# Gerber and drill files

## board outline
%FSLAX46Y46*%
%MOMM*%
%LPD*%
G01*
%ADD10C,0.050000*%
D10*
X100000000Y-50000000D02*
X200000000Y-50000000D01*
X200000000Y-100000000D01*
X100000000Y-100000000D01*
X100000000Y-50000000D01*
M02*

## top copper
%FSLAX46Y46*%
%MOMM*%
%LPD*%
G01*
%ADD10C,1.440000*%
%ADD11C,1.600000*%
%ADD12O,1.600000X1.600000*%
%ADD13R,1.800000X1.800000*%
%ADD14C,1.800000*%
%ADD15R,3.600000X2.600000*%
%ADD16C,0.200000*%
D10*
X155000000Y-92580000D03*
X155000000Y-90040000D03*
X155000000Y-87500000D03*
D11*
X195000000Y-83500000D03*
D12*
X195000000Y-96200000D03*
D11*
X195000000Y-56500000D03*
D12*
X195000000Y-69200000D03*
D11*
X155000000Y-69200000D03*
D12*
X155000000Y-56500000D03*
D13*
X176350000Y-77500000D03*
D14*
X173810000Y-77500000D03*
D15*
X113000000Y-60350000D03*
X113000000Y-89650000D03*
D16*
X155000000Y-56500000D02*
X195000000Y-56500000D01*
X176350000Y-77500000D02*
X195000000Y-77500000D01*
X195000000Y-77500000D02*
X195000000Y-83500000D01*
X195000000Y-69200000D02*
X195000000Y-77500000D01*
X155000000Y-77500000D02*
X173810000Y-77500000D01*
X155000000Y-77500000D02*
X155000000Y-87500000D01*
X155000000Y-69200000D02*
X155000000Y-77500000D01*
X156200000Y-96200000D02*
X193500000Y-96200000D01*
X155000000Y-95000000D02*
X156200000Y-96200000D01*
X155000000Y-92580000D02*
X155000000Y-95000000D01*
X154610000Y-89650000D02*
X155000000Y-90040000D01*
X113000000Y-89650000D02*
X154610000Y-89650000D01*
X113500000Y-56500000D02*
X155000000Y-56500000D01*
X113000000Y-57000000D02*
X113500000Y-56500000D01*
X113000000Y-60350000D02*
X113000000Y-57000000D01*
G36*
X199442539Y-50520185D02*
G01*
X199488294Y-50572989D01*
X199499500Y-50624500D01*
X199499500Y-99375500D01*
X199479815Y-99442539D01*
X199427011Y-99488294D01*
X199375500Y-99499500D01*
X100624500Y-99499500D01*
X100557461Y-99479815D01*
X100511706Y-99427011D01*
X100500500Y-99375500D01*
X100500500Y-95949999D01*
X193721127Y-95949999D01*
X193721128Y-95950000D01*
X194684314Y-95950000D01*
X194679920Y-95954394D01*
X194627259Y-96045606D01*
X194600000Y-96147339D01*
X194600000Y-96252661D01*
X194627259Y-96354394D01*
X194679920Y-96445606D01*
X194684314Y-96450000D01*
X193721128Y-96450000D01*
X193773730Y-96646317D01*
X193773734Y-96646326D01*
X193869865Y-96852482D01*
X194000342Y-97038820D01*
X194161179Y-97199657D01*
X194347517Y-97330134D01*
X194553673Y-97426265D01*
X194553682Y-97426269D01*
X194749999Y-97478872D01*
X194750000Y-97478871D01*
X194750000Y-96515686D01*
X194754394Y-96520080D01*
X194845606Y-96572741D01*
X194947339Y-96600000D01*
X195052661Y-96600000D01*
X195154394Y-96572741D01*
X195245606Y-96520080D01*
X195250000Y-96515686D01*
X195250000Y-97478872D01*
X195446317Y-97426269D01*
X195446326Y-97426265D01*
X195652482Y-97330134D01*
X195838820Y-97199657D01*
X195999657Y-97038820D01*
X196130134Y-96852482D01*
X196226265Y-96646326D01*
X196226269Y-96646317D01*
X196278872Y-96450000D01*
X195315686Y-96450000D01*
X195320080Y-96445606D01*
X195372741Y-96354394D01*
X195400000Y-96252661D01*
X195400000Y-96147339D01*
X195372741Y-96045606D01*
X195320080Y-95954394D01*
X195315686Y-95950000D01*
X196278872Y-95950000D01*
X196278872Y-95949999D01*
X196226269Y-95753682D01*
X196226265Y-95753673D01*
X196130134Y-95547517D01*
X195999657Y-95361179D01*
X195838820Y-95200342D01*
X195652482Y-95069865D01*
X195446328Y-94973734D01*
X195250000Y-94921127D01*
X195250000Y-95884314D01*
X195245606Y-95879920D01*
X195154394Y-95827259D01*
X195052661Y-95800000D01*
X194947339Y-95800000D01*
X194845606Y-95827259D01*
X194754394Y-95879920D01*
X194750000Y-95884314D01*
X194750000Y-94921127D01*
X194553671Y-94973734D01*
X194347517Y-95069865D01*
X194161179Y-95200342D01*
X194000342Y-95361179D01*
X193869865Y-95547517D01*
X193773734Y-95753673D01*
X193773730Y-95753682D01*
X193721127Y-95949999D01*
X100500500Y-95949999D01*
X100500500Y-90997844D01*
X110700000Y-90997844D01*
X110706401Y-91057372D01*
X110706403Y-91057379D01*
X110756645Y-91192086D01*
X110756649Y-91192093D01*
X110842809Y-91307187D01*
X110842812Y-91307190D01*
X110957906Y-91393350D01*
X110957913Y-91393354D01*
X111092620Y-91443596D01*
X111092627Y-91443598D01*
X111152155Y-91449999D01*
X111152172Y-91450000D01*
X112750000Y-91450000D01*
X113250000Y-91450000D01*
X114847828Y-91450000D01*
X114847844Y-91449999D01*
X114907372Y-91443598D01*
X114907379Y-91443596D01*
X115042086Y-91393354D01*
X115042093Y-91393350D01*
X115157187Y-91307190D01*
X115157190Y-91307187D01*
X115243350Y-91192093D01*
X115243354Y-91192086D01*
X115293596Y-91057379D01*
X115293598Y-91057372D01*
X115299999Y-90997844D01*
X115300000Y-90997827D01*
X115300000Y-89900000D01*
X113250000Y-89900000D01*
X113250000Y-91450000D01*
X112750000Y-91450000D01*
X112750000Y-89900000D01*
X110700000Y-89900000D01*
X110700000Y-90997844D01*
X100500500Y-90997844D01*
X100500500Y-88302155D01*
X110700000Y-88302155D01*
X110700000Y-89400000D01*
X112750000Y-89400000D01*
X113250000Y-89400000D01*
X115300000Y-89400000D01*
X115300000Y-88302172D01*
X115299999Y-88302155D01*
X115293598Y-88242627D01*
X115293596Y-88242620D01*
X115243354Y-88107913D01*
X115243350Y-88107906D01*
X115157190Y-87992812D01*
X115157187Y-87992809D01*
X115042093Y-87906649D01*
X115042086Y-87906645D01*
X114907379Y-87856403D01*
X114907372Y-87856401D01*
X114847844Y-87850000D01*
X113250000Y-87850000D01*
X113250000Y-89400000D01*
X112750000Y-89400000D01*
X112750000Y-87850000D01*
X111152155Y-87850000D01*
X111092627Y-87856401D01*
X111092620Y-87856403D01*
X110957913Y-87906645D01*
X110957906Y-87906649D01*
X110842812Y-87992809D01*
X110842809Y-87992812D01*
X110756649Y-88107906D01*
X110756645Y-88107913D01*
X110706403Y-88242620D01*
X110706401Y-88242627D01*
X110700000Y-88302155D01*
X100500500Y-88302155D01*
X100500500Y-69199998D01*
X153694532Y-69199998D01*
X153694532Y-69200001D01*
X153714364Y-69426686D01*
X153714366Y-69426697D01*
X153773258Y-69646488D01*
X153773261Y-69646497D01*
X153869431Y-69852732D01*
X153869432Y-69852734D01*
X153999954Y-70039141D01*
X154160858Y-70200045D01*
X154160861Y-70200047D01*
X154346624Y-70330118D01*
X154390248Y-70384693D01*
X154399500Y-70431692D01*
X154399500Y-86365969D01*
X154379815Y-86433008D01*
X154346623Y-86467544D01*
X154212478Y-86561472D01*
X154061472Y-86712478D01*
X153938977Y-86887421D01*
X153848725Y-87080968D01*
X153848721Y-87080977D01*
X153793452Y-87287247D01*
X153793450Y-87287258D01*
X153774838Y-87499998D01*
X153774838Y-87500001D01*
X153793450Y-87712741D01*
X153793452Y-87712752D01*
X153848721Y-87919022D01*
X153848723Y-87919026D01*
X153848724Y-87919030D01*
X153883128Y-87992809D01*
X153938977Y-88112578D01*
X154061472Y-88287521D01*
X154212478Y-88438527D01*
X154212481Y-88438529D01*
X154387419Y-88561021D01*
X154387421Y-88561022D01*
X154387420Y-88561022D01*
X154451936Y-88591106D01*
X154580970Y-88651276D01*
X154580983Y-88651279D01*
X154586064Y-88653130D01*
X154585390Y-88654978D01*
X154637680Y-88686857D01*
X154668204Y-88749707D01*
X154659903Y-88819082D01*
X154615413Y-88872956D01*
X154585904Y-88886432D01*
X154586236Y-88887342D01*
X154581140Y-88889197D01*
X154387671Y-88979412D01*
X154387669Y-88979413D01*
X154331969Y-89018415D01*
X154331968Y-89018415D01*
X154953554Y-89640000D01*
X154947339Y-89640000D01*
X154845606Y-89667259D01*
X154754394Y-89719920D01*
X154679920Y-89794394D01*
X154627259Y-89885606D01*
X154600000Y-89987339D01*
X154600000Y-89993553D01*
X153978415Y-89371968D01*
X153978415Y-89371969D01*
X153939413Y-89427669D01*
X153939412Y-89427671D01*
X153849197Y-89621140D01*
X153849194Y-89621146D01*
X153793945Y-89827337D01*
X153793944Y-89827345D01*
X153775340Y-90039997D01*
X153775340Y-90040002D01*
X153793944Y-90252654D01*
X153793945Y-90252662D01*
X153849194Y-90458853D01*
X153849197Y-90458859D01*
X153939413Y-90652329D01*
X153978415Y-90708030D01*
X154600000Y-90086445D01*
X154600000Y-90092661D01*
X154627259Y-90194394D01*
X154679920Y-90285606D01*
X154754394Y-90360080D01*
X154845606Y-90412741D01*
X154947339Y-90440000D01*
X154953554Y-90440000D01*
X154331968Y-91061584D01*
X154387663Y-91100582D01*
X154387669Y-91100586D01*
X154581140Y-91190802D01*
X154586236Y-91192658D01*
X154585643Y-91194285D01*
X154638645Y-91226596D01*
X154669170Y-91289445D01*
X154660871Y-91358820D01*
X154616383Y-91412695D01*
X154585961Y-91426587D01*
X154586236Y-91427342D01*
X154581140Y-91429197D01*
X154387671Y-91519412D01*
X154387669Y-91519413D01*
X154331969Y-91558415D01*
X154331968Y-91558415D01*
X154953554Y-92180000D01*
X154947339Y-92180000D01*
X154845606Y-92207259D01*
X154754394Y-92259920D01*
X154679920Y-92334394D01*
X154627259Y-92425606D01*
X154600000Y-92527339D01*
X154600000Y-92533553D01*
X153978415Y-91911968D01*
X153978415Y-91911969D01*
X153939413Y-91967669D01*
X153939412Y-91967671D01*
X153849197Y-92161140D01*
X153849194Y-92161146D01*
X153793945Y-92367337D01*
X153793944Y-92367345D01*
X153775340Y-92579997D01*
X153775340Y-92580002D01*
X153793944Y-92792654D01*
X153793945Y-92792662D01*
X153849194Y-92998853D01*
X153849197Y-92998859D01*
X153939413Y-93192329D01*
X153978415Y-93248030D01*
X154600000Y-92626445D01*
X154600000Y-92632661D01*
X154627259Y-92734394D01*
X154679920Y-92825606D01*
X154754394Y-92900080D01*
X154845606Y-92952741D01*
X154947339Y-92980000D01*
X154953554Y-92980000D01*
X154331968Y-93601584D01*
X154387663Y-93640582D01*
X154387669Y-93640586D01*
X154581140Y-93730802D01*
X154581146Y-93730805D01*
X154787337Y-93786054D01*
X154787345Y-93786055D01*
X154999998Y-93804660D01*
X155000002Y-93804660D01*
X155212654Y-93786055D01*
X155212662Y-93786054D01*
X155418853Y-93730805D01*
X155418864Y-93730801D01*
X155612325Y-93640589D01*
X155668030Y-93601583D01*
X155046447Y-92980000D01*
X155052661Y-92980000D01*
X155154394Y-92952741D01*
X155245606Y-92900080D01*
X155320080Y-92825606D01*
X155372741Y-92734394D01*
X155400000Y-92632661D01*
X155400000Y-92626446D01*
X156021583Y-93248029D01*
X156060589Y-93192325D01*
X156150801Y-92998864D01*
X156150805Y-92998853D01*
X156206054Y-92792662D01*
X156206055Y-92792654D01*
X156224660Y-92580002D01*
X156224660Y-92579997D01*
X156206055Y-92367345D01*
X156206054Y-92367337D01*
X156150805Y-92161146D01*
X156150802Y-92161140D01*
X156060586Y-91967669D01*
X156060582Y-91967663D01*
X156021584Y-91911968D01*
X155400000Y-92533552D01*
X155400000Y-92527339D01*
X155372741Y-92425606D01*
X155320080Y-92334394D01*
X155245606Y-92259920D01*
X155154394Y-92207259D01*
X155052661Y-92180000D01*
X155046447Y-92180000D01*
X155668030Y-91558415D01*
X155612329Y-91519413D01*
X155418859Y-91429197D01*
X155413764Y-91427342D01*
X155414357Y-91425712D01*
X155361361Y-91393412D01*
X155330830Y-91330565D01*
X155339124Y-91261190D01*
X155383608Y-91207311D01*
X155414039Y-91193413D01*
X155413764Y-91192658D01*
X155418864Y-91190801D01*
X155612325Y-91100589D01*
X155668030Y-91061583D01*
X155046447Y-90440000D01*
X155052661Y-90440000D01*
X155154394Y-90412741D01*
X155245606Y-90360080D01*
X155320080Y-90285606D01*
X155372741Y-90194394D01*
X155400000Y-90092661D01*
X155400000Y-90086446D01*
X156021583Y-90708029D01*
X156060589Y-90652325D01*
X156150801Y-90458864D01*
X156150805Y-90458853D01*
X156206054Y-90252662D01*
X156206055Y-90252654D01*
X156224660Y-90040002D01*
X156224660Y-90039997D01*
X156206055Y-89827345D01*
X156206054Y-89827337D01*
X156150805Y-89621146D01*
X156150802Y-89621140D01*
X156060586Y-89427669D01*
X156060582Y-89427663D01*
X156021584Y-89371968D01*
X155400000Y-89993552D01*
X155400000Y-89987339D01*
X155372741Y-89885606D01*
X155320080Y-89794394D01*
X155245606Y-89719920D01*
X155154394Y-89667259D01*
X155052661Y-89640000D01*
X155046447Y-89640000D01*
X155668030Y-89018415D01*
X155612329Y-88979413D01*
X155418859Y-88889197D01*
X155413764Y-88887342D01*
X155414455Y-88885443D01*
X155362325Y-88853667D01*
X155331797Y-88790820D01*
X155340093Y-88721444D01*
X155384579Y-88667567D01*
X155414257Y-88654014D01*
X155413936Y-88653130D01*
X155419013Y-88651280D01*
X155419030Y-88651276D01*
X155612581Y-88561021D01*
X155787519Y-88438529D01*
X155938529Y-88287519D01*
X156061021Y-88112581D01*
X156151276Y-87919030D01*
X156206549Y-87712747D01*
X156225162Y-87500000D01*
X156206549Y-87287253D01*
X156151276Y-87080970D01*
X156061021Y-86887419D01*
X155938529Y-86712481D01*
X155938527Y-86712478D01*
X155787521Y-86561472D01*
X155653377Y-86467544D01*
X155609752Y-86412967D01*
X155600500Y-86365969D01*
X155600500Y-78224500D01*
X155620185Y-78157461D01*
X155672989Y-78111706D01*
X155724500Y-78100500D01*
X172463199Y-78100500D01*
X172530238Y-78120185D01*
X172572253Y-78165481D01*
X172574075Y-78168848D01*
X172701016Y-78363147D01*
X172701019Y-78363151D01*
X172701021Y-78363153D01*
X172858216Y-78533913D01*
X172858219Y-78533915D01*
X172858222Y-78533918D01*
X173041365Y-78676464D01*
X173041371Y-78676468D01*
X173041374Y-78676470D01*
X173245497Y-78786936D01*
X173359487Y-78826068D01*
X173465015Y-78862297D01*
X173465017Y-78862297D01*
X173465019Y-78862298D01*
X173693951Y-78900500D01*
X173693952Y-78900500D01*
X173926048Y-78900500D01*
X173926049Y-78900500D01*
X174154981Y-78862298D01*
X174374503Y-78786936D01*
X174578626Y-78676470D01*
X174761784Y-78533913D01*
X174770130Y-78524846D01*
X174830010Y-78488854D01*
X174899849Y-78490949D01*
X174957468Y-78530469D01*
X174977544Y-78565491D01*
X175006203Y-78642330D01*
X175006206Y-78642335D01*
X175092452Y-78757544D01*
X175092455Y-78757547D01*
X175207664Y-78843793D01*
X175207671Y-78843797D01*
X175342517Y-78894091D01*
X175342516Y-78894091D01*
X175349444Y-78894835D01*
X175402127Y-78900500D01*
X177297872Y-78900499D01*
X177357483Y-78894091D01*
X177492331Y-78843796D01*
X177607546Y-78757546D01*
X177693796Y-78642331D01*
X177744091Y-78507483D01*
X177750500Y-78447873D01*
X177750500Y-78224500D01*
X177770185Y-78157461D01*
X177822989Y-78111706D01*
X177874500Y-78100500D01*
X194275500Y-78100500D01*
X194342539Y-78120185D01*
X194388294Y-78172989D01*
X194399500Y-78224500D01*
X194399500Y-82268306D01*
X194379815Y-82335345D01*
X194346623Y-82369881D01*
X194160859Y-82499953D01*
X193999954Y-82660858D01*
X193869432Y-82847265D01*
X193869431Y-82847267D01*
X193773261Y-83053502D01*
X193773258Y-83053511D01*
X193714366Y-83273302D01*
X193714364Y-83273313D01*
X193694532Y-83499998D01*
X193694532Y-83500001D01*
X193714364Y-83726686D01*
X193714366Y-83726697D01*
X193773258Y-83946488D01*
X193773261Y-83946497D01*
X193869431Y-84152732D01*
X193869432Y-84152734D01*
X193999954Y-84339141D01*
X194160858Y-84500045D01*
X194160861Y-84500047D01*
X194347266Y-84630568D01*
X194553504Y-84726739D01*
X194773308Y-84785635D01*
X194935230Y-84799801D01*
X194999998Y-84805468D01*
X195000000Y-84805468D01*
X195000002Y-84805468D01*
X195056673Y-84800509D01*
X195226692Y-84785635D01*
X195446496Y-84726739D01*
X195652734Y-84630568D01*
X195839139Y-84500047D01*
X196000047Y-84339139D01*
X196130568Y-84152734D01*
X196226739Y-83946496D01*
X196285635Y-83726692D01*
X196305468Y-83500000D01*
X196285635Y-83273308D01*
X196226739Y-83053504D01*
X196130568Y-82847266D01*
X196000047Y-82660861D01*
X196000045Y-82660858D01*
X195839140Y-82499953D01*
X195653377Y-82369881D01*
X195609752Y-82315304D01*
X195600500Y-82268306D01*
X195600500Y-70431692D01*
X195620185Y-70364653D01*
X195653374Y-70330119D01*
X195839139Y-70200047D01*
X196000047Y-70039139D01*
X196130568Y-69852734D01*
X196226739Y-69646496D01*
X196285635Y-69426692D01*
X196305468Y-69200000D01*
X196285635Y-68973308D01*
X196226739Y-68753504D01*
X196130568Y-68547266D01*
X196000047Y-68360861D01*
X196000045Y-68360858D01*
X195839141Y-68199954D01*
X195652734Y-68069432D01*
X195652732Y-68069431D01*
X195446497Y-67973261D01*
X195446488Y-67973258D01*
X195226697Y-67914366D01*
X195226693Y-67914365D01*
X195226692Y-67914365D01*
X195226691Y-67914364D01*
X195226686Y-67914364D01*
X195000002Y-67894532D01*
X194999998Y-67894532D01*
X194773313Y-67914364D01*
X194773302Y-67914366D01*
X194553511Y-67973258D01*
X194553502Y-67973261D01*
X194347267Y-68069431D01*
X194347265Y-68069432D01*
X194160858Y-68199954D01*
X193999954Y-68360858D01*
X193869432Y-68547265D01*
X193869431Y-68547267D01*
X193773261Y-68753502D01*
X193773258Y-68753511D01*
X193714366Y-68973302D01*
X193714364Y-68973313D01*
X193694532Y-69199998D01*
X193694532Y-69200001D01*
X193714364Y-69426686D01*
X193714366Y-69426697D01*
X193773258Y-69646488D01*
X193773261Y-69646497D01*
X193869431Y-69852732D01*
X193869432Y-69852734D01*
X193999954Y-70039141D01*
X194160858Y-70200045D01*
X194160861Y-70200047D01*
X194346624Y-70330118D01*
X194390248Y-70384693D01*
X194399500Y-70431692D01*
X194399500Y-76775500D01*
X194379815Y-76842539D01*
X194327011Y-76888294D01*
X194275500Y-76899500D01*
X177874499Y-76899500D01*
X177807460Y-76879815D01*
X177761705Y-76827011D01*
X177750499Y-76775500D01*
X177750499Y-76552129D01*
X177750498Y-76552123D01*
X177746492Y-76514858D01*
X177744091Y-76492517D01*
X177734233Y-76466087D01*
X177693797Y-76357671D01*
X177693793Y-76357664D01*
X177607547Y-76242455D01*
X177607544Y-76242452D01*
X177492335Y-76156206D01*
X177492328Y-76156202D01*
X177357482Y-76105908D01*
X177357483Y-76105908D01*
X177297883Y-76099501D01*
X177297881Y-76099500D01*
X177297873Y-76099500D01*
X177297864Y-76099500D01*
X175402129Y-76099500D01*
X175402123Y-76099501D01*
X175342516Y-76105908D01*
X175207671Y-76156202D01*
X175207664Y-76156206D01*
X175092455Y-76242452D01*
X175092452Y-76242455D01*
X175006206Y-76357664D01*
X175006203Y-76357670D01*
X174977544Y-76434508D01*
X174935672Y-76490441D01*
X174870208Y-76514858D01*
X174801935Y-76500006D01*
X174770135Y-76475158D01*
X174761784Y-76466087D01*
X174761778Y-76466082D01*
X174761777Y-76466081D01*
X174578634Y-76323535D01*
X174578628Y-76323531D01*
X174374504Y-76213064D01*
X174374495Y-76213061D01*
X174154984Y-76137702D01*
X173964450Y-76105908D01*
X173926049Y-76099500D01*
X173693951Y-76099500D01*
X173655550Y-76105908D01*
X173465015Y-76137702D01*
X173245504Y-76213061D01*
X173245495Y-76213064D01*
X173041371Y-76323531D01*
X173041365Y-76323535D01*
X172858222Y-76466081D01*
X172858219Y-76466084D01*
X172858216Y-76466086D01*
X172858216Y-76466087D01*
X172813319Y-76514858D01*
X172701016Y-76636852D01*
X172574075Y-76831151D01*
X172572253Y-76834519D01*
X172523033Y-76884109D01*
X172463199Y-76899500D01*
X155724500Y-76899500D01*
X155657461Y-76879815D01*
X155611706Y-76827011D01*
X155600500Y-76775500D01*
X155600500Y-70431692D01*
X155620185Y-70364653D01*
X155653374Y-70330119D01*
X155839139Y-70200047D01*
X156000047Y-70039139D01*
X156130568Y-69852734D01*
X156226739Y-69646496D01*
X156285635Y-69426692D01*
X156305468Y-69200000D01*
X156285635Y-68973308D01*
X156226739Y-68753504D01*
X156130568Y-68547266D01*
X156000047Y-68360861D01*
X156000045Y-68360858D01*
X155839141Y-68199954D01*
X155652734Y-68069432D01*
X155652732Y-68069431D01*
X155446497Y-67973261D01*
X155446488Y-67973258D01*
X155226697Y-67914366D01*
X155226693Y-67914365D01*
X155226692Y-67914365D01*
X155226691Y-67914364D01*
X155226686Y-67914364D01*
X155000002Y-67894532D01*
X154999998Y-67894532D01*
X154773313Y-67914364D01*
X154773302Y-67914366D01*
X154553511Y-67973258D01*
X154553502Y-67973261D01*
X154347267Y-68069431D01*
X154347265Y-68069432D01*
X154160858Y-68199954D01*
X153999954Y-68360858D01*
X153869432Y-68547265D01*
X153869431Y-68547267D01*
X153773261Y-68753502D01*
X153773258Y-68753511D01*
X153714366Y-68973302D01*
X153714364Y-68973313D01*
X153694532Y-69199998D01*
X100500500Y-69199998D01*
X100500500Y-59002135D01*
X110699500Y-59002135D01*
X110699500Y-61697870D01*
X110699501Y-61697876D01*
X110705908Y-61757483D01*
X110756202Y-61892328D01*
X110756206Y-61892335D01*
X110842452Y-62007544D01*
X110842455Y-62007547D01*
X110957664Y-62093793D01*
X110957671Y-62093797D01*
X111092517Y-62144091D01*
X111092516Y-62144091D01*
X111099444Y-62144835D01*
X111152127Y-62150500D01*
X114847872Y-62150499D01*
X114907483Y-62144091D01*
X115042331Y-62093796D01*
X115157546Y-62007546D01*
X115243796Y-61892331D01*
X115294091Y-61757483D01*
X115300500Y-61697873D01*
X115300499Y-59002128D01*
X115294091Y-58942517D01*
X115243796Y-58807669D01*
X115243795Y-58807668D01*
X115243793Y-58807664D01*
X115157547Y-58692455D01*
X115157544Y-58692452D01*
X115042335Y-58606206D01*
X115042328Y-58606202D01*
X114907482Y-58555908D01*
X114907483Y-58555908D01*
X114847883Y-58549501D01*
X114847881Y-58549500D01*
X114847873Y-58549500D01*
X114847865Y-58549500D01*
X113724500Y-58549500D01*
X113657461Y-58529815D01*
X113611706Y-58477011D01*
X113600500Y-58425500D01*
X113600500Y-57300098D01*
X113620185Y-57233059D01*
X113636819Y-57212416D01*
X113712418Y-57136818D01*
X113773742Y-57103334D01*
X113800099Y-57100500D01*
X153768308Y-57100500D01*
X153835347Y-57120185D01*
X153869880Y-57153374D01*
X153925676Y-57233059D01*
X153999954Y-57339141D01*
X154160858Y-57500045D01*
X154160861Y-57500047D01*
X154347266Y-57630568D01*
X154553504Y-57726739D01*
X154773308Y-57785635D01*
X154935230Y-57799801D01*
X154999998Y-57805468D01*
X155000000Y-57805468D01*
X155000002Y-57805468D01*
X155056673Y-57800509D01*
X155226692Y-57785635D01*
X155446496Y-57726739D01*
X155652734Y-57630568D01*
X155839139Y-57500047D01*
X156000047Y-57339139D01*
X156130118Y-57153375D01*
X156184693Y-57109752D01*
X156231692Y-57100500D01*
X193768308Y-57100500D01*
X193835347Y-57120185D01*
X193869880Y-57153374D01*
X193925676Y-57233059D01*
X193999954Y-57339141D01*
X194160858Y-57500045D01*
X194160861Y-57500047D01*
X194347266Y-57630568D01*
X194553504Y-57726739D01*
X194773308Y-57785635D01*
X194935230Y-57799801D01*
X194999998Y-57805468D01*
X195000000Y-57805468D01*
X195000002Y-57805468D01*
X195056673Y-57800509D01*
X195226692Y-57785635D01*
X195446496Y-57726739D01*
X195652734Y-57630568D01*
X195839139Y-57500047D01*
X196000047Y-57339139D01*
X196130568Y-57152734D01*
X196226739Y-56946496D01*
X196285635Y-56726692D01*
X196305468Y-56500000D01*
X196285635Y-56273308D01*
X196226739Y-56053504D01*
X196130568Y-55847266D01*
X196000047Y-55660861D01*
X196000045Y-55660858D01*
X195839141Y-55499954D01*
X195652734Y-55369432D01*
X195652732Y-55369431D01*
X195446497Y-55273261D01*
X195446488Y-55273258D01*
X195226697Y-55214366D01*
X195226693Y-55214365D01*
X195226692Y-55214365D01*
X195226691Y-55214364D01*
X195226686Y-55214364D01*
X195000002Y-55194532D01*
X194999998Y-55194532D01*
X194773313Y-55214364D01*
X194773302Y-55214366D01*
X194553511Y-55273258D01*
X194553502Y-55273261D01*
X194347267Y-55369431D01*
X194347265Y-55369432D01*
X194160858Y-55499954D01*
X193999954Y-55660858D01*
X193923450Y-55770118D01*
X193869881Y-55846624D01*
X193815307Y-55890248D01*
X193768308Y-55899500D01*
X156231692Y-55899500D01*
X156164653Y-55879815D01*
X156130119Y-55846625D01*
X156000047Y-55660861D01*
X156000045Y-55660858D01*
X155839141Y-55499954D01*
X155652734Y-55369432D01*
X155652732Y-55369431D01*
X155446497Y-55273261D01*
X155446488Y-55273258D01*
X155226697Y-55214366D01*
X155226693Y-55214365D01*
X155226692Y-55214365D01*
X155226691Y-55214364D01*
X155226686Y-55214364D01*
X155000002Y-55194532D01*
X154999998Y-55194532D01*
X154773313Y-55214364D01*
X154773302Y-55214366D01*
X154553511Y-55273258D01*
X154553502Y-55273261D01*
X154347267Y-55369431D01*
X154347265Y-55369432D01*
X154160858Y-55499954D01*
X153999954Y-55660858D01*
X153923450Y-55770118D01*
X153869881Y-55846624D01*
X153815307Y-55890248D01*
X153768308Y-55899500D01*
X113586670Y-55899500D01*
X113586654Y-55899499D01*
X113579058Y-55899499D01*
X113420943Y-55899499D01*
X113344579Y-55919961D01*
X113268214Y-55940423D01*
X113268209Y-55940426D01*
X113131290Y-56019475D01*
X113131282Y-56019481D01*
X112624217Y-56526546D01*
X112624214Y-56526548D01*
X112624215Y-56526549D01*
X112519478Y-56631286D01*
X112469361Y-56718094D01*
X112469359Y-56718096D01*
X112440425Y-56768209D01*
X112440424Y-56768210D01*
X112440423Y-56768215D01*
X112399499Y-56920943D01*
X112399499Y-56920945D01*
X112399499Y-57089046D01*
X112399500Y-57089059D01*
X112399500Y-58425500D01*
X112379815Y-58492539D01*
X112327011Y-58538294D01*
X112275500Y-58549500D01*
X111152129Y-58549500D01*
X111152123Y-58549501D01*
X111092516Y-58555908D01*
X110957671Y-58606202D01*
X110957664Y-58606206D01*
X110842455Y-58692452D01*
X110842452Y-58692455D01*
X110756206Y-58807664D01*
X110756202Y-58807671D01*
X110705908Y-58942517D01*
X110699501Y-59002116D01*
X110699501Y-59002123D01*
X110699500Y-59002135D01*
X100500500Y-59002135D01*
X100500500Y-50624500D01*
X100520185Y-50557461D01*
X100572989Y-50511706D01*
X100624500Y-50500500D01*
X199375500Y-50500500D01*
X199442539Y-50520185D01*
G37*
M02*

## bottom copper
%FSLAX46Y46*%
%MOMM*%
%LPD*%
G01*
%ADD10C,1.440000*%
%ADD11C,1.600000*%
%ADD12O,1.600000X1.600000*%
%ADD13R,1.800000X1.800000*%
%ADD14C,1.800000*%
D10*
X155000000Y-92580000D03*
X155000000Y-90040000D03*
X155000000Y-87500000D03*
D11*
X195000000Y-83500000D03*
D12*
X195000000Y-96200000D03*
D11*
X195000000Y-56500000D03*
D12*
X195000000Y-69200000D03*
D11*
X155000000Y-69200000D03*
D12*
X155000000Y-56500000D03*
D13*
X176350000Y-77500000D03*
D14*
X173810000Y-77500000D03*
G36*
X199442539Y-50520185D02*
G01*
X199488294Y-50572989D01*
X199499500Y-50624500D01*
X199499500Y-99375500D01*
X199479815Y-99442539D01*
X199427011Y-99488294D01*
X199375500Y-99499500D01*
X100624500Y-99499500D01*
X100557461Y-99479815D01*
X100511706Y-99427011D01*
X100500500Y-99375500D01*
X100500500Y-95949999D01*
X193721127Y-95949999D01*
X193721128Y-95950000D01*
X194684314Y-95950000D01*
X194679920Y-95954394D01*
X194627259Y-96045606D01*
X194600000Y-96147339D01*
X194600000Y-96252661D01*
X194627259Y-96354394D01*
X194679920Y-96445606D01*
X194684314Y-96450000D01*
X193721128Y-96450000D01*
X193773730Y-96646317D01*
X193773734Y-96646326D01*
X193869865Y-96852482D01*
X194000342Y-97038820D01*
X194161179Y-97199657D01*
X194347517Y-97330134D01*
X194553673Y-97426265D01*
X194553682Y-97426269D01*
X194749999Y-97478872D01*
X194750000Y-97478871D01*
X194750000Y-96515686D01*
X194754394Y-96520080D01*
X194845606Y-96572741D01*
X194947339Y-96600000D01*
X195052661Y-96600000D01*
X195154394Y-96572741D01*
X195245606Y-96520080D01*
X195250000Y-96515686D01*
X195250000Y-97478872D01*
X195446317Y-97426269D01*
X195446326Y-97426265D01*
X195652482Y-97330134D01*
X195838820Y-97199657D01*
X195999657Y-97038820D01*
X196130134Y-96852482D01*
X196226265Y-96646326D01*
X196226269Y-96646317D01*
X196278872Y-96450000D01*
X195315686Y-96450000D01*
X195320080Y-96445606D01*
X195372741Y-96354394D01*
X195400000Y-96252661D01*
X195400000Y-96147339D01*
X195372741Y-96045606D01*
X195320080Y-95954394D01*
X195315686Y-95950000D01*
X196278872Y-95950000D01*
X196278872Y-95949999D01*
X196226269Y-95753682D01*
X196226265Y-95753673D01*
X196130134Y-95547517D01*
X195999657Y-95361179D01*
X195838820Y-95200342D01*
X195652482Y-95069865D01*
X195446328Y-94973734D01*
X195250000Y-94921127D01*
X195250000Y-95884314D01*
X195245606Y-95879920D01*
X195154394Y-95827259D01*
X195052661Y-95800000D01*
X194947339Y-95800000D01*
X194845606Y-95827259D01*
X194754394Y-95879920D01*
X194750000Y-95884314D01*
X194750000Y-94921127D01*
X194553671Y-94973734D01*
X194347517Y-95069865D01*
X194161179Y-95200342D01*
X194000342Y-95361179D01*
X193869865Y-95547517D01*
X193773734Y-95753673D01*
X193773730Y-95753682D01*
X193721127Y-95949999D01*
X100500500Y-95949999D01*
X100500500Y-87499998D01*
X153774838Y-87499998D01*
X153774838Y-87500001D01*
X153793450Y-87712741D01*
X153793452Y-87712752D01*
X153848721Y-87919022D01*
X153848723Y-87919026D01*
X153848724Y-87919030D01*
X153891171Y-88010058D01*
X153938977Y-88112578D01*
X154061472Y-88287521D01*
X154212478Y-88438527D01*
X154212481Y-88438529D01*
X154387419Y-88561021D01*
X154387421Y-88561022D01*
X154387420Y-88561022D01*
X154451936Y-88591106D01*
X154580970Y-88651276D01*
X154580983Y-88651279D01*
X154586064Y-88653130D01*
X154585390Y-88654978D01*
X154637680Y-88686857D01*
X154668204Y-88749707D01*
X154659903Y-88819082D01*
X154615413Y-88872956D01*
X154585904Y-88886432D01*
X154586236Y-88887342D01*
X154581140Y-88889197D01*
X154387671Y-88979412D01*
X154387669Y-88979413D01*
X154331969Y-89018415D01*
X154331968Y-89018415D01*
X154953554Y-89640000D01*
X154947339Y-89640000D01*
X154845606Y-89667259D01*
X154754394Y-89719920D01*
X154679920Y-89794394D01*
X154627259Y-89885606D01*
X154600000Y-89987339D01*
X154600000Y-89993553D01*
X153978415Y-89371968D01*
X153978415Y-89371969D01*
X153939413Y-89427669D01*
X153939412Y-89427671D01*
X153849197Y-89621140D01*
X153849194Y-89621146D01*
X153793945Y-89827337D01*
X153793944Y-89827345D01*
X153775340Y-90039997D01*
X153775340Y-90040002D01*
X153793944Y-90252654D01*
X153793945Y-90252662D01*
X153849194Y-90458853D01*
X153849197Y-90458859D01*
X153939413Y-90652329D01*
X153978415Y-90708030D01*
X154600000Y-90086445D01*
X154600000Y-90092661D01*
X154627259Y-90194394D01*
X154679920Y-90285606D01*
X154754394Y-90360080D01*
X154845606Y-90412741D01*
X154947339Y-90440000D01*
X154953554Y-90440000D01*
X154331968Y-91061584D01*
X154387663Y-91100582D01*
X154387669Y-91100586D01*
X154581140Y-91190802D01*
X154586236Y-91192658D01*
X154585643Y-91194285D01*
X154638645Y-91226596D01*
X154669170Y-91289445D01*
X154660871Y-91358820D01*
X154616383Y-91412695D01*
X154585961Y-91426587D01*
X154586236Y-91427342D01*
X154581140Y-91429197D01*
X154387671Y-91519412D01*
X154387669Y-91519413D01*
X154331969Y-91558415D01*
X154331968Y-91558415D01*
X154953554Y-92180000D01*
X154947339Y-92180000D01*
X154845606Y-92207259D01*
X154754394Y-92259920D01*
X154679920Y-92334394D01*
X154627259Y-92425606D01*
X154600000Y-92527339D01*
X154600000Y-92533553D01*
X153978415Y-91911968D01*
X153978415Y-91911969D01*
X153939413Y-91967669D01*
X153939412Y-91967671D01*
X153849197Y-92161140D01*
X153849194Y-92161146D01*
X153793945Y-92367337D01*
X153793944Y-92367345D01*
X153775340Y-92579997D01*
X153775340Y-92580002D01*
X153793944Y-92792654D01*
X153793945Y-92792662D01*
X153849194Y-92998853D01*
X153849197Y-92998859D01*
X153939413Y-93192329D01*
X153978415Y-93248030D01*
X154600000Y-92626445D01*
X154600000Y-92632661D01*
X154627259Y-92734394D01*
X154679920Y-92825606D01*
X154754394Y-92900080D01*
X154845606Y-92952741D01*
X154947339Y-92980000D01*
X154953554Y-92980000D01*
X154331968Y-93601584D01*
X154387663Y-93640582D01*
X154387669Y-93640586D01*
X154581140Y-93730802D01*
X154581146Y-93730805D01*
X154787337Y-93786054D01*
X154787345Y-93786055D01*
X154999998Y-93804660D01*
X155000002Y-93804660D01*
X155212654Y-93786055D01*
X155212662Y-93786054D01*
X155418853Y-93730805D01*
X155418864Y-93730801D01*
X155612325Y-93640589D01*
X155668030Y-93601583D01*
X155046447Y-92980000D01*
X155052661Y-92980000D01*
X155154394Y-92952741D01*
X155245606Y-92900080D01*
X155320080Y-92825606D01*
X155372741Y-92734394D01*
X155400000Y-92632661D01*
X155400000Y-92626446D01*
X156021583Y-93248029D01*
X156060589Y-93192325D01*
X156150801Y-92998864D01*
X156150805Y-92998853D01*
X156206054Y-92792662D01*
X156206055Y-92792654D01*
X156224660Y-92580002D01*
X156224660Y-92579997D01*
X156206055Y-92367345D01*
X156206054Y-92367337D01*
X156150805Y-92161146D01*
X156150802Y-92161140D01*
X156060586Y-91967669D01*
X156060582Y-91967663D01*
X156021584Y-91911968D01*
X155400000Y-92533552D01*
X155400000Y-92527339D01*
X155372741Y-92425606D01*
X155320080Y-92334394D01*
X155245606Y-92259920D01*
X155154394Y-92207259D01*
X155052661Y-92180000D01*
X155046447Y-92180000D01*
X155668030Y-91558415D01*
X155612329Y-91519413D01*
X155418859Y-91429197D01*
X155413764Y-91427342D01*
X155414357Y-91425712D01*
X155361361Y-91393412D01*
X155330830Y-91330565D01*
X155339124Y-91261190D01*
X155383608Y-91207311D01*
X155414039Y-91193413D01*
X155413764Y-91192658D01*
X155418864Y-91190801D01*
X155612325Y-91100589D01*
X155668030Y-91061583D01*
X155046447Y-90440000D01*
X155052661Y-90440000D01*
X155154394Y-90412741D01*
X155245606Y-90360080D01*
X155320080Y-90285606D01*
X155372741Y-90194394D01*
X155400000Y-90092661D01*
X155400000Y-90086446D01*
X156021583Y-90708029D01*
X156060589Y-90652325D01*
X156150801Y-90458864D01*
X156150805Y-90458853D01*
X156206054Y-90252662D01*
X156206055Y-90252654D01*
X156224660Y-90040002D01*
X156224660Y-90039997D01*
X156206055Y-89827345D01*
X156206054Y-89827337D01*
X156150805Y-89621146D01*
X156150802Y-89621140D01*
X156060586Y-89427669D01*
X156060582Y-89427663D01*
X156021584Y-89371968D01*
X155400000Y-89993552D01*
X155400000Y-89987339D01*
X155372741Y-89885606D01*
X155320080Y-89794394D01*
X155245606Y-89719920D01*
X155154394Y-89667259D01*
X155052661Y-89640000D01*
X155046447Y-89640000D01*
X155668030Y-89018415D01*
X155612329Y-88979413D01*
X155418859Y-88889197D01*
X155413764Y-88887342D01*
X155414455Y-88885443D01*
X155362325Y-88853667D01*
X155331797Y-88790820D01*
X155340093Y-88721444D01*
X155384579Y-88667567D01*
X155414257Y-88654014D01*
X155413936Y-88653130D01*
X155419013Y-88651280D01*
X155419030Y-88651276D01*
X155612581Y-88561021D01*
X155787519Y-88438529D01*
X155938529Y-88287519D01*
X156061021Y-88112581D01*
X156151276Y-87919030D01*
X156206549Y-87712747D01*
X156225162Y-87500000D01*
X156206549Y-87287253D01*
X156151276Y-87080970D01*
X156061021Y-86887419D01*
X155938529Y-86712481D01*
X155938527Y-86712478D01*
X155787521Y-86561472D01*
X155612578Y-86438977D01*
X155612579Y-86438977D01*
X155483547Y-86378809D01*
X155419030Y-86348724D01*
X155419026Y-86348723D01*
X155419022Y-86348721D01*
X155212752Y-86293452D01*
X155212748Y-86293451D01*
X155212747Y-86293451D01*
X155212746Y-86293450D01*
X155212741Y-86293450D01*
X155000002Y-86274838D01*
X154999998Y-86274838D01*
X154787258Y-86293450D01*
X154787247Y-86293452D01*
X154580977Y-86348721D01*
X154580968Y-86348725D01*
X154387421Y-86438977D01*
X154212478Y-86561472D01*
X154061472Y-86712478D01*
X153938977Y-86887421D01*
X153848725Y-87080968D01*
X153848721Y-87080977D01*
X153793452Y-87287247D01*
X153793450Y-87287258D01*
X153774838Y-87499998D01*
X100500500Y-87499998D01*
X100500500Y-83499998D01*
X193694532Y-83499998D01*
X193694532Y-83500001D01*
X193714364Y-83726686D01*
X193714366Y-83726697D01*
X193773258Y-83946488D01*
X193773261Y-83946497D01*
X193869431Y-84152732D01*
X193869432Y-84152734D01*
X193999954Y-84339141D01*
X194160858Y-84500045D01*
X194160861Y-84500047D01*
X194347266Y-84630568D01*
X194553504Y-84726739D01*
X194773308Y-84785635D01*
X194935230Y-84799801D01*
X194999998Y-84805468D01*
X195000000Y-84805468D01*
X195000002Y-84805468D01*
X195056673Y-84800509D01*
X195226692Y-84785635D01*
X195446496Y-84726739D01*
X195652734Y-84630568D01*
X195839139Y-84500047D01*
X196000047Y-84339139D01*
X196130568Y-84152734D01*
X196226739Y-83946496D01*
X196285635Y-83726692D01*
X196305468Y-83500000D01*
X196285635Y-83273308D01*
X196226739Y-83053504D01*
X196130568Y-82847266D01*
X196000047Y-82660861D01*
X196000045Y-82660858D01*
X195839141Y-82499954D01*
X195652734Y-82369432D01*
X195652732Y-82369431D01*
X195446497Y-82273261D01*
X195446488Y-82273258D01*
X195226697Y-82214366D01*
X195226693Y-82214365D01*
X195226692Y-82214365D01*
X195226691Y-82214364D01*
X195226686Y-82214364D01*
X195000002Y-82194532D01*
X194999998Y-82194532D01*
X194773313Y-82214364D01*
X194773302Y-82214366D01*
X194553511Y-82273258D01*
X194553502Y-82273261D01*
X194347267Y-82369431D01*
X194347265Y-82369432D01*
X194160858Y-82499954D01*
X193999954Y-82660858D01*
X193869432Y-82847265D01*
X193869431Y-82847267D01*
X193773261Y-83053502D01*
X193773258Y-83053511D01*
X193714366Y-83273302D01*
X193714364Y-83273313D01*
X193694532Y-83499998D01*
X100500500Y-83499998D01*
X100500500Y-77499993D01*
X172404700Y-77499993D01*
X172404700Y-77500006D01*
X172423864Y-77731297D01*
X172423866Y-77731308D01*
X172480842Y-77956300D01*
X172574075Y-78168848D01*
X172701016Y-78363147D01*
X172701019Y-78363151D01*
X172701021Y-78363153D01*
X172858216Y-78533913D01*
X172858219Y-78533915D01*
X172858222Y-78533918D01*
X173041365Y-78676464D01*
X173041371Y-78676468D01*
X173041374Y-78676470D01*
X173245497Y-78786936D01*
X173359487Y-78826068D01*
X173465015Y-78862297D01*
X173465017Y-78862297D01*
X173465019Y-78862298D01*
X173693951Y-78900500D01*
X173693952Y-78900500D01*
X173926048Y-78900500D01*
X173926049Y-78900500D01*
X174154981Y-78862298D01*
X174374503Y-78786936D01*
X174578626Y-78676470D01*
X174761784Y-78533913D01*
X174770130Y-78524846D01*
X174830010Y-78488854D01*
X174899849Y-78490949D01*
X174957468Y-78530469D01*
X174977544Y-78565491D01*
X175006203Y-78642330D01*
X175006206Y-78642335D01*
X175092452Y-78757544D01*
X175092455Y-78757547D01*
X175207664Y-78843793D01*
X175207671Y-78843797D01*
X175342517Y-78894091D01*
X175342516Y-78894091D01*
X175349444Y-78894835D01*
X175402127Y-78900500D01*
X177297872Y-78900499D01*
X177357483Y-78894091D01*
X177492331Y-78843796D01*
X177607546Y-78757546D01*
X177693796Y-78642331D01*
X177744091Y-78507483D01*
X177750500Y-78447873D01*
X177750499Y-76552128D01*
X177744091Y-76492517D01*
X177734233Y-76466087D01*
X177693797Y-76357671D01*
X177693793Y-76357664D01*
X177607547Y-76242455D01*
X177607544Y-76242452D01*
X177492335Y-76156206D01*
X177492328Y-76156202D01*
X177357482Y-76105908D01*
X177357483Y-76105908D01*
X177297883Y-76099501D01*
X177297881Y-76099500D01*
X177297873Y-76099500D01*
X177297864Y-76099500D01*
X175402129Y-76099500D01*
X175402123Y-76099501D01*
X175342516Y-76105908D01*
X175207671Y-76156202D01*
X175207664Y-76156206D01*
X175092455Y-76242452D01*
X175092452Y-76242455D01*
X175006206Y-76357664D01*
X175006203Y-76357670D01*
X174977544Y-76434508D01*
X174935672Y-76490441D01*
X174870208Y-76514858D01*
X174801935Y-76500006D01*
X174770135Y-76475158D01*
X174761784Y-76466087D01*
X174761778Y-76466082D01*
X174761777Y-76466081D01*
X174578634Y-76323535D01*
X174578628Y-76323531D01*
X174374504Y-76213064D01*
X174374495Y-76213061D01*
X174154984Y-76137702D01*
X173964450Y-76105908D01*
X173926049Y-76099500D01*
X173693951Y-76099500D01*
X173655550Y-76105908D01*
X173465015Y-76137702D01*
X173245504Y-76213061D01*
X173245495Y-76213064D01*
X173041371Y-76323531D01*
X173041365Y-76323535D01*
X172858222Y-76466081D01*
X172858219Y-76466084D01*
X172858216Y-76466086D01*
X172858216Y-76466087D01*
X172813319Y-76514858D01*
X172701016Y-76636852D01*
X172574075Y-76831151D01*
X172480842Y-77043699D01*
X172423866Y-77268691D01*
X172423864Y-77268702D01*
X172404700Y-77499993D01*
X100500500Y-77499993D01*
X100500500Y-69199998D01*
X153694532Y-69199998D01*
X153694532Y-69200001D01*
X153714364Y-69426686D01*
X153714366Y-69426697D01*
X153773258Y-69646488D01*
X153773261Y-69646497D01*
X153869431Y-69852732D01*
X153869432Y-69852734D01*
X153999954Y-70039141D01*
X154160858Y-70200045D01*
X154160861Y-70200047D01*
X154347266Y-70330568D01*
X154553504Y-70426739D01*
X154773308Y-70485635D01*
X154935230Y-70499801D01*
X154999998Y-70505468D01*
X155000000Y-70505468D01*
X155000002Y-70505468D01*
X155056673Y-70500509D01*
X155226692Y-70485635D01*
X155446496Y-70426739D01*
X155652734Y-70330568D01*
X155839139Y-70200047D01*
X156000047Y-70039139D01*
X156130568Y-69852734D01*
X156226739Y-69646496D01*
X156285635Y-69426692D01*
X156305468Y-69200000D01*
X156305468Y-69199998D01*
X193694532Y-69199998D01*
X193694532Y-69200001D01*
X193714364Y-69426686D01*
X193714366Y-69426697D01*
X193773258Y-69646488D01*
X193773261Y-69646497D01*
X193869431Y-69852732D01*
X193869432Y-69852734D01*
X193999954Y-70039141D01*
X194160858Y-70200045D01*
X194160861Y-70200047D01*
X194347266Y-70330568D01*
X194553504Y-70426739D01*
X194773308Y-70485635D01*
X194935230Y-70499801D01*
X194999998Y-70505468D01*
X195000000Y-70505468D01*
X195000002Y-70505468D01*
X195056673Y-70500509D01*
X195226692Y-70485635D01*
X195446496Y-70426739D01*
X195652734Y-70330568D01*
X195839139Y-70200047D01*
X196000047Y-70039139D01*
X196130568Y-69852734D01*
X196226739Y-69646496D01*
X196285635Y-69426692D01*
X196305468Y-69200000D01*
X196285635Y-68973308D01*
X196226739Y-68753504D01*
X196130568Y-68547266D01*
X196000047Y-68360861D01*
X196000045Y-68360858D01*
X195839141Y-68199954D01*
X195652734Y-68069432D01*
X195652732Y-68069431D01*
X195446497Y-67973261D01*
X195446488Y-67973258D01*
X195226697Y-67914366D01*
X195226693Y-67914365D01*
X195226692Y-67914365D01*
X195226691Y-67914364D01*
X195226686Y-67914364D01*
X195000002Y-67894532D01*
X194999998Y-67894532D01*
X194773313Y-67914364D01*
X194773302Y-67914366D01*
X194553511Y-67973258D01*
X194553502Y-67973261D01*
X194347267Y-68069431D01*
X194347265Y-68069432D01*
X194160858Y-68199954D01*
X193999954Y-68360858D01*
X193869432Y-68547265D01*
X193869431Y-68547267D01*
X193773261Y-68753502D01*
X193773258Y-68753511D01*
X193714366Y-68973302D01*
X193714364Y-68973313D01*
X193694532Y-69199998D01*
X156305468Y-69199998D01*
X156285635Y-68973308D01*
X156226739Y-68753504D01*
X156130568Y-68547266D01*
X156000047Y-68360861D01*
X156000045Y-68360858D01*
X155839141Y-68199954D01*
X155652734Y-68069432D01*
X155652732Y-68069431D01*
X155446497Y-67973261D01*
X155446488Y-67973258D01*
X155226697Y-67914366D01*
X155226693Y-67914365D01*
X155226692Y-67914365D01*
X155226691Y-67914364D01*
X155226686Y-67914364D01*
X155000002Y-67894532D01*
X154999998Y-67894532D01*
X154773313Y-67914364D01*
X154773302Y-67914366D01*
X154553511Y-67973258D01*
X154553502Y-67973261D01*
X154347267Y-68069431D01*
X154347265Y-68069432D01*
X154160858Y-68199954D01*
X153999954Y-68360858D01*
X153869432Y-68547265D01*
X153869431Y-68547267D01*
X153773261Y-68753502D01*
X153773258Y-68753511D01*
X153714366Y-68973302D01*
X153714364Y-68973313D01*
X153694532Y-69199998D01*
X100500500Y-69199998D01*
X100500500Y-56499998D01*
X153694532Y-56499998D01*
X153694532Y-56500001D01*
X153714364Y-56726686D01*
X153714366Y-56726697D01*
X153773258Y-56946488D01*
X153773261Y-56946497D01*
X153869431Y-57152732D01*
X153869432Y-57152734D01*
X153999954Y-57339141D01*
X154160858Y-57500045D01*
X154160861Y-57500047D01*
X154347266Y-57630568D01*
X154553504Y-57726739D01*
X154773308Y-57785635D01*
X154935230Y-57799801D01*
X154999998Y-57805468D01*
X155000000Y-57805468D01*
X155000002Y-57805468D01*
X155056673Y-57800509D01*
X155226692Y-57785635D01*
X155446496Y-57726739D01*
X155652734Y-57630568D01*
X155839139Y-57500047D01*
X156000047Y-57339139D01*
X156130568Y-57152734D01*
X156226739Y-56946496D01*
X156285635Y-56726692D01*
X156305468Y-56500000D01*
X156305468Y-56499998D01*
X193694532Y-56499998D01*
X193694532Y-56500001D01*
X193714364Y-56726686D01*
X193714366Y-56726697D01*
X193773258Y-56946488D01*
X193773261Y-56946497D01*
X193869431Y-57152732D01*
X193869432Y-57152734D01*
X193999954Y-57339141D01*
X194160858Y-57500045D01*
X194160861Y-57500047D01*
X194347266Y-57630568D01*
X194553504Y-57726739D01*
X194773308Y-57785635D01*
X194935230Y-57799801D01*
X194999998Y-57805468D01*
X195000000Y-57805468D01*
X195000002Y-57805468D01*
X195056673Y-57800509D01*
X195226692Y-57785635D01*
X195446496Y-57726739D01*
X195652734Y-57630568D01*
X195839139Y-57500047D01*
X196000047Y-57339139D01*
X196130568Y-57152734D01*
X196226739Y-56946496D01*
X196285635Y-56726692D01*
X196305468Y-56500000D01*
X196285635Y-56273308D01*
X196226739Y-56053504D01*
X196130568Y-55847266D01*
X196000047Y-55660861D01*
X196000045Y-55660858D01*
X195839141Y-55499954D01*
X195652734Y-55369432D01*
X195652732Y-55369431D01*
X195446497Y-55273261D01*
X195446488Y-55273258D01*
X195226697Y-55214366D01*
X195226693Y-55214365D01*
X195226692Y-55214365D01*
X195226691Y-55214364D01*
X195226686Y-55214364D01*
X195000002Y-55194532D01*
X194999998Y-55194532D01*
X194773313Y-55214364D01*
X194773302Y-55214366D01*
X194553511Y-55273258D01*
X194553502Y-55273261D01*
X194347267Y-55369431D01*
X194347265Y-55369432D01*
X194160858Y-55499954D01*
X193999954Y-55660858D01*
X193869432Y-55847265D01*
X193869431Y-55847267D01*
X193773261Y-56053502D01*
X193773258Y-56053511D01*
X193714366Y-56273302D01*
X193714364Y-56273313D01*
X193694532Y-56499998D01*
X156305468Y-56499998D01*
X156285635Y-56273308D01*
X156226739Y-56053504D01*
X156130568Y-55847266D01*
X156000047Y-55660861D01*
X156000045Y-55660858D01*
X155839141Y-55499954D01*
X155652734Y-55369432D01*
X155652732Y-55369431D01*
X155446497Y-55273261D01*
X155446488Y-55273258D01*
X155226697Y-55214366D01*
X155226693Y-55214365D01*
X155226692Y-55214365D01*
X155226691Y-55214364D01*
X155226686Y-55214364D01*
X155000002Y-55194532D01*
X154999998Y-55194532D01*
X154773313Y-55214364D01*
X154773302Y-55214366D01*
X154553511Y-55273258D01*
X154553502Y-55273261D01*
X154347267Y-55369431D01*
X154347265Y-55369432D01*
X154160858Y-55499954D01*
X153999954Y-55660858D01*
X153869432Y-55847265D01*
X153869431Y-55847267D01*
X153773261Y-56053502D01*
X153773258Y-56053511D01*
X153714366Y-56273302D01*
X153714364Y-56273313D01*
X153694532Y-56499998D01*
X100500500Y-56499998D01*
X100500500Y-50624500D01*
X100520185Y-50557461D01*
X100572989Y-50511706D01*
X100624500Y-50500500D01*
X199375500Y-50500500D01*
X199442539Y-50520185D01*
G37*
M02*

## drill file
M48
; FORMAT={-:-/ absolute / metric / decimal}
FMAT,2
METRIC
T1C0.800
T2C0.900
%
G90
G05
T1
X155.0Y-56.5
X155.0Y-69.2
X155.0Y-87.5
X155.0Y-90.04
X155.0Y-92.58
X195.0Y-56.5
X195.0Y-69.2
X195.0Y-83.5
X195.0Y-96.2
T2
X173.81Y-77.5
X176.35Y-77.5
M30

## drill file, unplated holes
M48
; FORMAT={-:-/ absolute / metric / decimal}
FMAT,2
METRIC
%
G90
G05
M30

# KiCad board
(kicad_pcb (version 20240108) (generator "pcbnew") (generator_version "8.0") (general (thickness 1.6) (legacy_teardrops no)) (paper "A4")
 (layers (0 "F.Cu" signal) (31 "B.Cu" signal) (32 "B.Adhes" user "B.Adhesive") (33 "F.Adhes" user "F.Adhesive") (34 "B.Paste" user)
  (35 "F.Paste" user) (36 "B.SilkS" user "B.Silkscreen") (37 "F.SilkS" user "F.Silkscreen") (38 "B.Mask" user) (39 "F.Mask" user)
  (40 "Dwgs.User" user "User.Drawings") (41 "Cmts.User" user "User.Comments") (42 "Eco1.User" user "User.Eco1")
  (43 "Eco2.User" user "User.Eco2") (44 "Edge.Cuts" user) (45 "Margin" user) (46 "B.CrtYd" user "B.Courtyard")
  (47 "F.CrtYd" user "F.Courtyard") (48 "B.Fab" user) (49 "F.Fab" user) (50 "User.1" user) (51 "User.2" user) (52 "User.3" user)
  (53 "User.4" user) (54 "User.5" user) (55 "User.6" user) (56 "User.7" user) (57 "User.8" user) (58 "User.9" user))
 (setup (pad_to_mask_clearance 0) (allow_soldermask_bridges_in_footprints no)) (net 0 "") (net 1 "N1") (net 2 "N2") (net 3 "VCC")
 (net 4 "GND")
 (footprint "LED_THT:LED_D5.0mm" (layer "F.Cu") (at 176.35 77.5 180)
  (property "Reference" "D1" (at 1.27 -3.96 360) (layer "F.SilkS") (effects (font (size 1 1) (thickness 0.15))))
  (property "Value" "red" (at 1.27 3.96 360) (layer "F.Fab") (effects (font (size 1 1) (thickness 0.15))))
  (pad "1" thru_hole rect (at 0 0 180) (size 1.8 1.8) (drill 0.9) (layers "*.Cu" "*.Mask") (remove_unused_layers no) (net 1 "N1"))
  (pad "2" thru_hole circle (at 2.54 0 180) (size 1.8 1.8) (drill 0.9) (layers "*.Cu" "*.Mask") (remove_unused_layers no) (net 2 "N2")))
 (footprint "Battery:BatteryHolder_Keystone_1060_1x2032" (layer "F.Cu") (at 113 75 -90)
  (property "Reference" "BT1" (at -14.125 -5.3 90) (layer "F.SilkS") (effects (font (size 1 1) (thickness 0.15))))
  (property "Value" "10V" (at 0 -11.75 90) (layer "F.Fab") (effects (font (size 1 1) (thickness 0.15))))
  (pad "1" smd rect (at -14.65 0 90) (size 2.6 3.6) (layers "F.Cu" "F.Paste" "F.Mask") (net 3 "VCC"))
  (pad "2" smd rect (at 14.65 0 90) (size 2.6 3.6) (layers "F.Cu" "F.Paste" "F.Mask") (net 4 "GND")))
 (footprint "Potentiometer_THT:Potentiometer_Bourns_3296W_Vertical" (layer "F.Cu") (at 155 92.58 -90)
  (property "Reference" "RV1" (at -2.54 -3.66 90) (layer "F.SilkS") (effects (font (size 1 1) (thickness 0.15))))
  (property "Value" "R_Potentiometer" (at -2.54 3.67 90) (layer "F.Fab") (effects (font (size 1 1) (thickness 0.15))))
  (pad "1" thru_hole circle (at 0 0 270) (size 1.44 1.44) (drill 0.8) (layers "*.Cu" "*.Mask") (remove_unused_layers no) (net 4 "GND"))
  (pad "2" thru_hole circle (at -2.54 0 270) (size 1.44 1.44) (drill 0.8) (layers "*.Cu" "*.Mask") (remove_unused_layers no) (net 4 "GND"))
  (pad "3" thru_hole circle (at -5.08 0 270) (size 1.44 1.44) (drill 0.8) (layers "*.Cu" "*.Mask") (remove_unused_layers no) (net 2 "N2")))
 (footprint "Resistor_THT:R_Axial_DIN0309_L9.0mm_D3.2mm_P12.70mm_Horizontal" (layer "F.Cu") (at 155 69.2 90)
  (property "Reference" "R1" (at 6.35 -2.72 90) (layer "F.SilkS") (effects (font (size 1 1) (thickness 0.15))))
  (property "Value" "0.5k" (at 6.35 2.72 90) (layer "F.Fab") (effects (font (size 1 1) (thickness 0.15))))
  (pad "1" thru_hole circle (at 0 0 90) (size 1.6 1.6) (drill 0.8) (layers "*.Cu" "*.Mask") (remove_unused_layers no) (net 2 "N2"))
  (pad "2" thru_hole oval (at 12.7 0 90) (size 1.6 1.6) (drill 0.8) (layers "*.Cu" "*.Mask") (remove_unused_layers no) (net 3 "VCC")))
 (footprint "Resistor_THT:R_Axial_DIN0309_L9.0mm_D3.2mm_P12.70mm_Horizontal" (layer "F.Cu") (at 195 83.5 -90)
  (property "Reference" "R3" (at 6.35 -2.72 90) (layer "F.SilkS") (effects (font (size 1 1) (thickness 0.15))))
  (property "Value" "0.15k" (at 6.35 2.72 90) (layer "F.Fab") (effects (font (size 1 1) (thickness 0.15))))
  (pad "1" thru_hole circle (at 0 0 270) (size 1.6 1.6) (drill 0.8) (layers "*.Cu" "*.Mask") (remove_unused_layers no) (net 1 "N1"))
  (pad "2" thru_hole oval (at 12.7 0 270) (size 1.6 1.6) (drill 0.8) (layers "*.Cu" "*.Mask") (remove_unused_layers no) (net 4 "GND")))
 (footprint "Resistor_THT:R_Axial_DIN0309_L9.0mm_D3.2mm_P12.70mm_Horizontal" (layer "F.Cu") (at 195 56.5 -90)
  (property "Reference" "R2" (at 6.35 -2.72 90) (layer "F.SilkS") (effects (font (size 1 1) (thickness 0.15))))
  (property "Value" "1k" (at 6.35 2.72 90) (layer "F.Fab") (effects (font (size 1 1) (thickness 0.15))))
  (pad "1" thru_hole circle (at 0 0 270) (size 1.6 1.6) (drill 0.8) (layers "*.Cu" "*.Mask") (remove_unused_layers no) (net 3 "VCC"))
  (pad "2" thru_hole oval (at 12.7 0 270) (size 1.6 1.6) (drill 0.8) (layers "*.Cu" "*.Mask") (remove_unused_layers no) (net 1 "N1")))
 (gr_rect (start 100 50) (end 200 100) (stroke (width 0.05) (type default)) (fill none) (layer "Edge.Cuts"))
 (segment (start 156.2 96.2) (end 193.5 96.2) (width 0.2) (layer "F.Cu") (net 4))
 (segment (start 155 95) (end 156.2 96.2) (width 0.2) (layer "F.Cu") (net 4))
 (segment (start 155 92.58) (end 155 95) (width 0.2) (layer "F.Cu") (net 4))
 (segment (start 113 89.65) (end 154.61 89.65) (width 0.2) (layer "F.Cu") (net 4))
 (segment (start 154.61 89.65) (end 155 90.04) (width 0.2) (layer "F.Cu") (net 4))
 (segment (start 155 56.5) (end 195 56.5) (width 0.2) (layer "F.Cu") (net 3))
 (segment (start 113 57) (end 113.5 56.5) (width 0.2) (layer "F.Cu") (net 3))
 (segment (start 113 60.35) (end 113 57) (width 0.2) (layer "F.Cu") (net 3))
 (segment (start 113.5 56.5) (end 155 56.5) (width 0.2) (layer "F.Cu") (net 3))
 (segment (start 195 77.5) (end 195 83.5) (width 0.2) (layer "F.Cu") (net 1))
 (segment (start 195 69.2) (end 195 77.5) (width 0.2) (layer "F.Cu") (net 1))
 (segment (start 176.35 77.5) (end 195 77.5) (width 0.2) (layer "F.Cu") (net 1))
 (segment (start 155 69.2) (end 155 77.5) (width 0.2) (layer "F.Cu") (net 2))
 (segment (start 155 77.5) (end 173.81 77.5) (width 0.2) (layer "F.Cu") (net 2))
 (segment (start 155 77.5) (end 155 87.5) (width 0.2) (layer "F.Cu") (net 2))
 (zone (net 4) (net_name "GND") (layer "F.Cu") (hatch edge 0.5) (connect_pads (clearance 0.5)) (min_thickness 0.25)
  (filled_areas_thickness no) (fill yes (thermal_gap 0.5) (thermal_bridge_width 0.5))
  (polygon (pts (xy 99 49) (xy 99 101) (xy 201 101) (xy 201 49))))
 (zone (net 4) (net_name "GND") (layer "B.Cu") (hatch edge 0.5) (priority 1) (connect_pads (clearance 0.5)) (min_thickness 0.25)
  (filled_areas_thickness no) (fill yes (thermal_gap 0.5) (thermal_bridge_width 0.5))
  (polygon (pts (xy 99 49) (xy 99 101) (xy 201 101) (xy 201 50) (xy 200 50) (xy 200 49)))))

